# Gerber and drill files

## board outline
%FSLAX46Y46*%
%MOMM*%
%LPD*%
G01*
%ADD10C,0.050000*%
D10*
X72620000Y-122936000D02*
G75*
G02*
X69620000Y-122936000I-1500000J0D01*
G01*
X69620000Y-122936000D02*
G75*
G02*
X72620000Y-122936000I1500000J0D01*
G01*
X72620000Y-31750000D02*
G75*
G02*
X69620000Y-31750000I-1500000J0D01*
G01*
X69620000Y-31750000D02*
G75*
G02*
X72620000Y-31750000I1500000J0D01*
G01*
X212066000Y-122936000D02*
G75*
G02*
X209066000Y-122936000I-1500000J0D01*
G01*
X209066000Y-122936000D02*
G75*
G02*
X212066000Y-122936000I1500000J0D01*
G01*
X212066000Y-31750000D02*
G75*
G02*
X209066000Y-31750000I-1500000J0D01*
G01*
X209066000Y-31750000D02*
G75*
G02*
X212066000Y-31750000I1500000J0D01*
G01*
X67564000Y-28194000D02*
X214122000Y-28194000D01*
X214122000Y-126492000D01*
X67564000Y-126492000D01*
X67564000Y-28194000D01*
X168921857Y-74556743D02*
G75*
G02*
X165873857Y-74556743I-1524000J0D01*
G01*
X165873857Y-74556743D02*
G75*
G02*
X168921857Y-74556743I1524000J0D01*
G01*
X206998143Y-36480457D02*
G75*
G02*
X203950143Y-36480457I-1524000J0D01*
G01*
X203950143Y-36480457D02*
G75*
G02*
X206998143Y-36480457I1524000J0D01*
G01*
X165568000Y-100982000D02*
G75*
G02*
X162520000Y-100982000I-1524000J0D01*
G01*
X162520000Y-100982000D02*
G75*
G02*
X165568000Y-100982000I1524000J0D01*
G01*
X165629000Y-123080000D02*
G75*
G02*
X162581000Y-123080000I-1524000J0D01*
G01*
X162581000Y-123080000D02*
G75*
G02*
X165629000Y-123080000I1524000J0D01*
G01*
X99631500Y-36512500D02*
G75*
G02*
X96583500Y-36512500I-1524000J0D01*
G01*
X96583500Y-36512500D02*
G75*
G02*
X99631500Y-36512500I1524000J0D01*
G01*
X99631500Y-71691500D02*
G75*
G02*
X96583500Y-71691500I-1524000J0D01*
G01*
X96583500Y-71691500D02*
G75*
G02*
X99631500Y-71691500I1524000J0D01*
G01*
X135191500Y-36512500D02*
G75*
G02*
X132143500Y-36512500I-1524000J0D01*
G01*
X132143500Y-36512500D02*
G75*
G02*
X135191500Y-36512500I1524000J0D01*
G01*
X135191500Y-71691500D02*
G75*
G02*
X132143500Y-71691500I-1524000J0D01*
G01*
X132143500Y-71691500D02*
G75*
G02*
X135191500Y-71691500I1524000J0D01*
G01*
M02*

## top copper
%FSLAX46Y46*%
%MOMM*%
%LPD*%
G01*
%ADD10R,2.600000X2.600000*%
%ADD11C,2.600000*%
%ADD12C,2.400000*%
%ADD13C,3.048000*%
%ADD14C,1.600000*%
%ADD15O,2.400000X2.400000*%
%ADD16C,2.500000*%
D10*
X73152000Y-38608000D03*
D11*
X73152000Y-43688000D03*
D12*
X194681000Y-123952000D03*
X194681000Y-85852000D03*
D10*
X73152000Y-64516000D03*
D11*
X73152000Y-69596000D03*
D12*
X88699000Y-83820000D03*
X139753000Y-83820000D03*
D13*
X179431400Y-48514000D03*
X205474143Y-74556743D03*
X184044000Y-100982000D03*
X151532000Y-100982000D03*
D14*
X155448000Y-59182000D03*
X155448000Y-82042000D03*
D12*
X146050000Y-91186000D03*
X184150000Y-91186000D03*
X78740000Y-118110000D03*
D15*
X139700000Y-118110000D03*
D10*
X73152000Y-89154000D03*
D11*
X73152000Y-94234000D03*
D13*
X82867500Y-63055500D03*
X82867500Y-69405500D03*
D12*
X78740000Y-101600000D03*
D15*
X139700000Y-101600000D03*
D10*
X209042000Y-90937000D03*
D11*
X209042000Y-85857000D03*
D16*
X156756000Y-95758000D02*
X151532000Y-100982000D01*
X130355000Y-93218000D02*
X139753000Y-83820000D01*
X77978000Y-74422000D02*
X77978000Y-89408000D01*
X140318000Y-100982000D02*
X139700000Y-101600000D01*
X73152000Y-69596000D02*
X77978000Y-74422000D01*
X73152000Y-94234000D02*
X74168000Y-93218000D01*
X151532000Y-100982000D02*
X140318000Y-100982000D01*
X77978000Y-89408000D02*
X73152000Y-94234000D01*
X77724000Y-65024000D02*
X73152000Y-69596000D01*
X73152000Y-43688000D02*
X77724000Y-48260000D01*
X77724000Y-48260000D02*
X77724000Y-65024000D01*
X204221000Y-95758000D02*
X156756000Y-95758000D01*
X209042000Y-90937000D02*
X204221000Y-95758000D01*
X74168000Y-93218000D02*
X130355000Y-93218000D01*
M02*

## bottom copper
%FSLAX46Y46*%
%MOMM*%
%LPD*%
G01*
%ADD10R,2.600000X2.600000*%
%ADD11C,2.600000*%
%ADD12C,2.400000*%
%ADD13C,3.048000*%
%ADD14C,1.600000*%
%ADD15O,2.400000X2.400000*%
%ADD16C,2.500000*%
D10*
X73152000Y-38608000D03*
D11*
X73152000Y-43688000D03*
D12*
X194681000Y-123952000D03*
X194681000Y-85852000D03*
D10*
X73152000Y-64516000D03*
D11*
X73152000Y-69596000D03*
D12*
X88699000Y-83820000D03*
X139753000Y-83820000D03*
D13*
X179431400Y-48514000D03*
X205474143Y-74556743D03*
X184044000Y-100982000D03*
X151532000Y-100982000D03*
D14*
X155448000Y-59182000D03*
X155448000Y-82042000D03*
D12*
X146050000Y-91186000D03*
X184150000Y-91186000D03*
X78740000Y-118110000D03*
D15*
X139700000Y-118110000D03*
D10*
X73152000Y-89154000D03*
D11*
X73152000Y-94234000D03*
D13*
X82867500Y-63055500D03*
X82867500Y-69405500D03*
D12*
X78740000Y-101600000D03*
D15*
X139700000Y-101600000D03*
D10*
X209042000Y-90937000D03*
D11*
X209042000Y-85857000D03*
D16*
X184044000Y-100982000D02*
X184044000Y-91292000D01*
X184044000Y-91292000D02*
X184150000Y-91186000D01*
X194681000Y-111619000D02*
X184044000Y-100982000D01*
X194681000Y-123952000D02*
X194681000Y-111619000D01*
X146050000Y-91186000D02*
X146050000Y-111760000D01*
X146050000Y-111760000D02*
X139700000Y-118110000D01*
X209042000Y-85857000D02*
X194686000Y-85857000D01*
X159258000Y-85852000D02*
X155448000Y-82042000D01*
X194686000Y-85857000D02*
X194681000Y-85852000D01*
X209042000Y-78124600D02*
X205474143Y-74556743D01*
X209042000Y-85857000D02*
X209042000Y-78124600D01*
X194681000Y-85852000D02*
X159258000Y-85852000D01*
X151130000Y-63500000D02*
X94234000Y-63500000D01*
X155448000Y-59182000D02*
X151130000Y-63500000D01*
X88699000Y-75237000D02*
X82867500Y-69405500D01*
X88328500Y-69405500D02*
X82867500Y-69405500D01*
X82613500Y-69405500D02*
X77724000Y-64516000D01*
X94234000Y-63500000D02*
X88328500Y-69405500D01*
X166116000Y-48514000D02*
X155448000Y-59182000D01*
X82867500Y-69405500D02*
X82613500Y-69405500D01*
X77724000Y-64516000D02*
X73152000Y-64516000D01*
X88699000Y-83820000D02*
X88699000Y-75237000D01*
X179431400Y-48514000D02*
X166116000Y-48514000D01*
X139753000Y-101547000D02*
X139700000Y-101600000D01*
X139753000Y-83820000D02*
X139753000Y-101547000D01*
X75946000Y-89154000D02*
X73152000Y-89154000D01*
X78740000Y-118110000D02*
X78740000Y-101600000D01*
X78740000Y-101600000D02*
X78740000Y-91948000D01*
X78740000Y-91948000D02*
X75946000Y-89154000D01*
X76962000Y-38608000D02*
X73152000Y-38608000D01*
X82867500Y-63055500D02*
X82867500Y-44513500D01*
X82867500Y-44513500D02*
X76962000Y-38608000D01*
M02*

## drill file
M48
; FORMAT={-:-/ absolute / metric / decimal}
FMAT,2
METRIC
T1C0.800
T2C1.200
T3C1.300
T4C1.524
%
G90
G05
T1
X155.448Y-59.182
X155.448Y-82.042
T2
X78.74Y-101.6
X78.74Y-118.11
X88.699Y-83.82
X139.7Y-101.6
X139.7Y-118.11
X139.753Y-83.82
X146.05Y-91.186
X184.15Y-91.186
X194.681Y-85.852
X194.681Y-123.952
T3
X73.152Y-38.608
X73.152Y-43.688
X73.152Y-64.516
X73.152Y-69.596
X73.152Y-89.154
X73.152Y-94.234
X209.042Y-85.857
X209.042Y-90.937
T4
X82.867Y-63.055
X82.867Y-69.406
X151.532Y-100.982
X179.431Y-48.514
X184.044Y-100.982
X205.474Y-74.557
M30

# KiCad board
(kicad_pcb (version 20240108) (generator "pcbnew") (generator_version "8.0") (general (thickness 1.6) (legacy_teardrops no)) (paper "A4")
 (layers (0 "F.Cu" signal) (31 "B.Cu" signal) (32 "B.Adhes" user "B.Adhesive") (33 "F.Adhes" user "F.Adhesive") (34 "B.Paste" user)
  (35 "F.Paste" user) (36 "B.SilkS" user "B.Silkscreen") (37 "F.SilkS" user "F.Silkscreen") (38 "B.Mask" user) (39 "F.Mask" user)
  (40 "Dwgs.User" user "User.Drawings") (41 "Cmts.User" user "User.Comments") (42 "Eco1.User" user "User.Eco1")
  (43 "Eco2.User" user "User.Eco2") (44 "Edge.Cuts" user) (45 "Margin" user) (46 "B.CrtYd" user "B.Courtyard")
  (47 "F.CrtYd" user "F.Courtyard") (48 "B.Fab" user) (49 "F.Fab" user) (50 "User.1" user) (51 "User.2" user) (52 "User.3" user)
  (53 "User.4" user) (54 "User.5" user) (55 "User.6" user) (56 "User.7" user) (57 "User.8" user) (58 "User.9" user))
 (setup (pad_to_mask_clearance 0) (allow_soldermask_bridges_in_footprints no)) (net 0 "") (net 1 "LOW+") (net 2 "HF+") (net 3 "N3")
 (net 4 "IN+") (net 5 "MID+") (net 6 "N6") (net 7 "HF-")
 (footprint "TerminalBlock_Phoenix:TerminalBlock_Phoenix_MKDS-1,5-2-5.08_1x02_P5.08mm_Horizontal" (layer "F.Cu") (at 73.152 38.608 -90)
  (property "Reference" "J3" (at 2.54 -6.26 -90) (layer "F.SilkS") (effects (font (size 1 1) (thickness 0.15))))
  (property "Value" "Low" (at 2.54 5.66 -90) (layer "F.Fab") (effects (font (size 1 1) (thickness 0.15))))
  (pad "1" thru_hole rect (at 0 0 270) (size 2.6 2.6) (drill 1.3) (layers "*.Cu" "*.Mask") (remove_unused_layers no) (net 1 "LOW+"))
  (pad "2" thru_hole circle (at 5.08 0 270) (size 2.6 2.6) (drill 1.3) (layers "*.Cu" "*.Mask") (remove_unused_layers no) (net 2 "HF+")))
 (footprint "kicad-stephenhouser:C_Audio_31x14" (layer "F.Cu") (at 194.681 123.952 90)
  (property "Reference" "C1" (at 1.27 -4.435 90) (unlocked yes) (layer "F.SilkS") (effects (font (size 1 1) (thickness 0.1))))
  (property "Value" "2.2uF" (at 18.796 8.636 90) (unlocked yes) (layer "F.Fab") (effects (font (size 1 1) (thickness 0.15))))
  (pad "1" thru_hole circle (at 0 0 90) (size 2.4 2.4) (drill 1.2) (layers "*.Cu" "*.Mask") (remove_unused_layers no) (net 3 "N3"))
  (pad "2" thru_hole circle (at 38.1 0 90) (size 2.4 2.4) (drill 1.2) (layers "*.Cu" "*.Mask") (remove_unused_layers no) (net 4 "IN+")))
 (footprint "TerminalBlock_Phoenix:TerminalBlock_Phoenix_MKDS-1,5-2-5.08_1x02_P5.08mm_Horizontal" (layer "F.Cu") (at 73.152 64.516 -90)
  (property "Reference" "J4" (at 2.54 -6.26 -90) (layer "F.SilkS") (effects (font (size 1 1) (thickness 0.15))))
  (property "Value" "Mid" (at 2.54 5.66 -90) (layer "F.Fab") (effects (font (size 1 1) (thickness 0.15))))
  (pad "1" thru_hole rect (at 0 0 270) (size 2.6 2.6) (drill 1.3) (layers "*.Cu" "*.Mask") (remove_unused_layers no) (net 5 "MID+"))
  (pad "2" thru_hole circle (at 5.08 0 270) (size 2.6 2.6) (drill 1.3) (layers "*.Cu" "*.Mask") (remove_unused_layers no) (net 2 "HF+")))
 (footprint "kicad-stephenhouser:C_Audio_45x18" (layer "F.Cu") (at 88.699 83.82)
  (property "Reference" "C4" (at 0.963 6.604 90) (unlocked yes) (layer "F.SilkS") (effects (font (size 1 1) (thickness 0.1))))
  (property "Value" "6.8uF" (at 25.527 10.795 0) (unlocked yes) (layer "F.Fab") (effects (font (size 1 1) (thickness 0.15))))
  (pad "1" thru_hole circle (at 0 0) (size 2.4 2.4) (drill 1.2) (layers "*.Cu" "*.Mask") (remove_unused_layers no) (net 5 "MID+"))
  (pad "2" thru_hole circle (at 51.054 0) (size 2.4 2.4) (drill 1.2) (layers "*.Cu" "*.Mask") (remove_unused_layers no) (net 2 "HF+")))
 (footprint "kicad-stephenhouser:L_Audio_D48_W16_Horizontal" (layer "F.Cu") (at 186.436 55.5186 -45)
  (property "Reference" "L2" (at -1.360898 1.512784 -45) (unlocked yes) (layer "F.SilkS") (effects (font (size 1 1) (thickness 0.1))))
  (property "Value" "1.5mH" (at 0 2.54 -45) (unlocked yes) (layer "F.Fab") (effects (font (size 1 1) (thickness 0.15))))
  (fp_circle (center 0 26.924) (end 1.524 26.924) (stroke (width 0.05) (type default)) (fill none) (layer "Edge.Cuts"))
  (fp_circle (center 0 -26.924) (end 1.524 -26.924) (stroke (width 0.05) (type default)) (fill none) (layer "Edge.Cuts"))
  (pad "1" thru_hole circle (at -9.906 0 315) (size 3.048 3.048) (drill 1.524) (layers "*.Cu" "*.Mask") (remove_unused_layers no)
   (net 5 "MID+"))
  (pad "2" thru_hole circle (at 26.924 0 315) (size 3.048 3.048) (drill 1.524) (layers "*.Cu" "*.Mask") (remove_unused_layers no)
   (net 4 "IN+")))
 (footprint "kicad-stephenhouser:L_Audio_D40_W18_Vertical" (layer "F.Cu") (at 184.044 100.982 180)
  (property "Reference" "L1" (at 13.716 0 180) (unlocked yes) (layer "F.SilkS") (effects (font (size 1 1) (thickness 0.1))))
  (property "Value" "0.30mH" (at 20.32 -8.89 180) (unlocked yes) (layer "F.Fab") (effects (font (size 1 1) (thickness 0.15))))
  (fp_circle (center 20 0) (end 21.524 0) (stroke (width 0.05) (type default)) (fill none) (layer "Edge.Cuts"))
  (fp_circle (center 19.939 -22.098) (end 21.463 -22.098) (stroke (width 0.05) (type default)) (fill none) (layer "Edge.Cuts"))
  (pad "1" thru_hole circle (at 0 0 180) (size 3.048 3.048) (drill 1.524) (layers "*.Cu" "*.Mask") (remove_unused_layers no) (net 3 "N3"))
  (pad "2" thru_hole circle (at 32.512 0 180) (size 3.048 3.048) (drill 1.524) (layers "*.Cu" "*.Mask") (remove_unused_layers no)
   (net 2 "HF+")))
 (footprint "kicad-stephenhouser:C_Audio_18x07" (layer "F.Cu") (at 155.448 59.182 -90)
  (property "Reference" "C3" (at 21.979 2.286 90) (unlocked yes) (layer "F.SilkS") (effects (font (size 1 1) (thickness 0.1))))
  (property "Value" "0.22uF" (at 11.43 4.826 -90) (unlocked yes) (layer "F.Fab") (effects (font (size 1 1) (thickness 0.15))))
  (pad "1" thru_hole circle (at 0 0 270) (size 1.6 1.6) (drill 0.8) (layers "*.Cu" "*.Mask") (remove_unused_layers no) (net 5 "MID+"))
  (pad "2" thru_hole circle (at 22.86 0 270) (size 1.6 1.6) (drill 0.8) (layers "*.Cu" "*.Mask") (remove_unused_layers no) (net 4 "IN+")))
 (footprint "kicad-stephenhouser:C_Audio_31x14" (layer "F.Cu") (at 146.05 91.186)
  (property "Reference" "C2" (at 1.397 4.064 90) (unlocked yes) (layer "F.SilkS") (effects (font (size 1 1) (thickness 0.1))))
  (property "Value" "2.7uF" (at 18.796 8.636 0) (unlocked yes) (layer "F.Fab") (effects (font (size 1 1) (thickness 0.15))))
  (pad "1" thru_hole circle (at 0 0) (size 2.4 2.4) (drill 1.2) (layers "*.Cu" "*.Mask") (remove_unused_layers no) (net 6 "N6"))
  (pad "2" thru_hole circle (at 38.1 0) (size 2.4 2.4) (drill 1.2) (layers "*.Cu" "*.Mask") (remove_unused_layers no) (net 3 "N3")))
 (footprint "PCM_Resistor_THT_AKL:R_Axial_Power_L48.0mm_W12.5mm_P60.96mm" (layer "F.Cu") (at 78.74 118.11)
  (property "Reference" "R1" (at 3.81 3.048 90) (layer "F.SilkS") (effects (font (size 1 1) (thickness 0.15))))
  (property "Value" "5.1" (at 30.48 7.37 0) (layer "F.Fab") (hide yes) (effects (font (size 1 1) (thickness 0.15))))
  (pad "1" thru_hole circle (at 0 0) (size 2.4 2.4) (drill 1.2) (layers "*.Cu" "*.Mask") (remove_unused_layers no) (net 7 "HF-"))
  (pad "2" thru_hole oval (at 60.96 0) (size 2.4 2.4) (drill 1.2) (layers "*.Cu" "*.Mask") (remove_unused_layers no) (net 6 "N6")))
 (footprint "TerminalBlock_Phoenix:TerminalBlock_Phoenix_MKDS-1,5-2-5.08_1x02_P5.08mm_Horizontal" (layer "F.Cu") (at 73.152 89.154 -90)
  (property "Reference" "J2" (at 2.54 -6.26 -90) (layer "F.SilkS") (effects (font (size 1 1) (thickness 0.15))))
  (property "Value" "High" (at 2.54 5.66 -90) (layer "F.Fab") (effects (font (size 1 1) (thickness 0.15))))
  (pad "1" thru_hole rect (at 0 0 270) (size 2.6 2.6) (drill 1.3) (layers "*.Cu" "*.Mask") (remove_unused_layers no) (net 7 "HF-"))
  (pad "2" thru_hole circle (at 5.08 0 270) (size 2.6 2.6) (drill 1.3) (layers "*.Cu" "*.Mask") (remove_unused_layers no) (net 2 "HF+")))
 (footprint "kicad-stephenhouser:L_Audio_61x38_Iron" (layer "F.Cu") (at 82.8675 69.4055)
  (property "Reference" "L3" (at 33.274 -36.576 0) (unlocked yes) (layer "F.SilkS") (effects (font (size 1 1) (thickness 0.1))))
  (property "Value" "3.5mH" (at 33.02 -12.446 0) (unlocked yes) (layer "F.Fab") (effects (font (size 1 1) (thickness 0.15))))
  (fp_circle (center 15.24 -32.893) (end 16.764 -32.893) (stroke (width 0.05) (type default)) (fill none) (layer "Edge.Cuts"))
  (fp_circle (center 15.24 2.286) (end 16.764 2.286) (stroke (width 0.05) (type default)) (fill none) (layer "Edge.Cuts"))
  (fp_circle (center 50.8 -32.893) (end 52.324 -32.893) (stroke (width 0.05) (type default)) (fill none) (layer "Edge.Cuts"))
  (fp_circle (center 50.8 2.286) (end 52.324 2.286) (stroke (width 0.05) (type default)) (fill none) (layer "Edge.Cuts"))
  (pad "1" thru_hole circle (at 0 -6.35) (size 3.048 3.048) (drill 1.524) (layers "*.Cu" "*.Mask") (remove_unused_layers no) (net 1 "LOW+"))
  (pad "2" thru_hole circle (at 0 0) (size 3.048 3.048) (drill 1.524) (layers "*.Cu" "*.Mask") (remove_unused_layers no) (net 5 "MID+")))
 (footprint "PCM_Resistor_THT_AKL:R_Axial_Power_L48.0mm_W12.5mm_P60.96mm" (layer "F.Cu") (at 78.74 101.6)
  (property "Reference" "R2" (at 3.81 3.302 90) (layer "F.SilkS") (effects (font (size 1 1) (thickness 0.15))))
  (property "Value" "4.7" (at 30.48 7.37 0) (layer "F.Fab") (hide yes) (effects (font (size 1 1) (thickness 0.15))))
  (pad "1" thru_hole circle (at 0 0) (size 2.4 2.4) (drill 1.2) (layers "*.Cu" "*.Mask") (remove_unused_layers no) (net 7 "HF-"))
  (pad "2" thru_hole oval (at 60.96 0) (size 2.4 2.4) (drill 1.2) (layers "*.Cu" "*.Mask") (remove_unused_layers no) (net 2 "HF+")))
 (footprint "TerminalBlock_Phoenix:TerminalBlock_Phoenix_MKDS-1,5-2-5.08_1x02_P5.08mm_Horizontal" (layer "F.Cu") (at 209.042 90.937 90)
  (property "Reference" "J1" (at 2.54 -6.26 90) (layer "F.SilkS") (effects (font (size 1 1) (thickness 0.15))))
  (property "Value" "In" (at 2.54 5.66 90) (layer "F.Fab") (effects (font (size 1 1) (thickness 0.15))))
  (pad "1" thru_hole rect (at 0 0 90) (size 2.6 2.6) (drill 1.3) (layers "*.Cu" "*.Mask") (remove_unused_layers no) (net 2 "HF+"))
  (pad "2" thru_hole circle (at 5.08 0 90) (size 2.6 2.6) (drill 1.3) (layers "*.Cu" "*.Mask") (remove_unused_layers no) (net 4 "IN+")))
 (gr_circle (center 71.12 122.936) (end 72.62 122.936) (stroke (width 0.05) (type default)) (fill none) (layer "Edge.Cuts"))
 (gr_circle (center 71.12 31.75) (end 72.62 31.75) (stroke (width 0.05) (type default)) (fill none) (layer "Edge.Cuts"))
 (gr_circle (center 210.566 122.936) (end 212.066 122.936) (stroke (width 0.05) (type default)) (fill none) (layer "Edge.Cuts"))
 (gr_circle (center 210.566 31.75) (end 212.066 31.75) (stroke (width 0.05) (type default)) (fill none) (layer "Edge.Cuts"))
 (gr_rect (start 67.564 28.194) (end 214.122 126.492) (stroke (width 0.05) (type default)) (fill none) (layer "Edge.Cuts"))
 (segment (start 184.044 100.982) (end 184.044 91.292) (width 2.5) (layer "B.Cu") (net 3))
 (segment (start 184.044 91.292) (end 184.15 91.186) (width 2.5) (layer "B.Cu") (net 3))
 (segment (start 194.681 111.619) (end 184.044 100.982) (width 2.5) (layer "B.Cu") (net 3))
 (segment (start 194.681 123.952) (end 194.681 111.619) (width 2.5) (layer "B.Cu") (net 3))
 (segment (start 146.05 91.186) (end 146.05 111.76) (width 2.5) (layer "B.Cu") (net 6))
 (segment (start 146.05 111.76) (end 139.7 118.11) (width 2.5) (layer "B.Cu") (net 6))
 (segment (start 209.042 85.857) (end 194.686 85.857) (width 2.5) (layer "B.Cu") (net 4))
 (segment (start 159.258 85.852) (end 155.448 82.042) (width 2.5) (layer "B.Cu") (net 4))
 (segment (start 194.686 85.857) (end 194.681 85.852) (width 2.5) (layer "B.Cu") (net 4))
 (segment (start 209.042 78.1246) (end 205.474143 74.556743) (width 2.5) (layer "B.Cu") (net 4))
 (segment (start 209.042 85.857) (end 209.042 78.1246) (width 2.5) (layer "B.Cu") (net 4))
 (segment (start 194.681 85.852) (end 159.258 85.852) (width 2.5) (layer "B.Cu") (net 4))
 (segment (start 151.13 63.5) (end 94.234 63.5) (width 2.5) (layer "B.Cu") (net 5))
 (segment (start 155.448 59.182) (end 151.13 63.5) (width 2.5) (layer "B.Cu") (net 5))
 (segment (start 88.699 75.237) (end 82.8675 69.4055) (width 2.5) (layer "B.Cu") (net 5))
 (segment (start 88.3285 69.4055) (end 82.8675 69.4055) (width 2.5) (layer "B.Cu") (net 5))
 (segment (start 82.6135 69.4055) (end 77.724 64.516) (width 2.5) (layer "B.Cu") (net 5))
 (segment (start 94.234 63.5) (end 88.3285 69.4055) (width 2.5) (layer "B.Cu") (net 5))
 (segment (start 166.116 48.514) (end 155.448 59.182) (width 2.5) (layer "B.Cu") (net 5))
 (segment (start 82.8675 69.4055) (end 82.6135 69.4055) (width 2.5) (layer "B.Cu") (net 5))
 (segment (start 77.724 64.516) (end 73.152 64.516) (width 2.5) (layer "B.Cu") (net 5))
 (segment (start 88.699 83.82) (end 88.699 75.237) (width 2.5) (layer "B.Cu") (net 5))
 (segment (start 179.4314 48.514) (end 166.116 48.514) (width 2.5) (layer "B.Cu") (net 5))
 (segment (start 156.756 95.758) (end 151.532 100.982) (width 2.5) (layer "F.Cu") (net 2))
 (segment (start 130.355 93.218) (end 139.753 83.82) (width 2.5) (layer "F.Cu") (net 2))
 (segment (start 77.978 74.422) (end 77.978 89.408) (width 2.5) (layer "F.Cu") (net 2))
 (segment (start 140.318 100.982) (end 139.7 101.6) (width 2.5) (layer "F.Cu") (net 2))
 (segment (start 73.152 69.596) (end 77.978 74.422) (width 2.5) (layer "F.Cu") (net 2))
 (segment (start 73.152 94.234) (end 74.168 93.218) (width 2.5) (layer "F.Cu") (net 2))
 (segment (start 151.532 100.982) (end 140.318 100.982) (width 2.5) (layer "F.Cu") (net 2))
 (segment (start 77.978 89.408) (end 73.152 94.234) (width 2.5) (layer "F.Cu") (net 2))
 (segment (start 77.724 65.024) (end 73.152 69.596) (width 2.5) (layer "F.Cu") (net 2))
 (segment (start 73.152 43.688) (end 77.724 48.26) (width 2.5) (layer "F.Cu") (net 2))
 (segment (start 77.724 48.26) (end 77.724 65.024) (width 2.5) (layer "F.Cu") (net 2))
 (segment (start 204.221 95.758) (end 156.756 95.758) (width 2.5) (layer "F.Cu") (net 2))
 (segment (start 209.042 90.937) (end 204.221 95.758) (width 2.5) (layer "F.Cu") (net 2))
 (segment (start 74.168 93.218) (end 130.355 93.218) (width 2.5) (layer "F.Cu") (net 2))
 (segment (start 139.753 101.547) (end 139.7 101.6) (width 2.5) (layer "B.Cu") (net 2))
 (segment (start 139.753 83.82) (end 139.753 101.547) (width 2.5) (layer "B.Cu") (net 2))
 (segment (start 75.946 89.154) (end 73.152 89.154) (width 2.5) (layer "B.Cu") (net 7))
 (segment (start 78.74 118.11) (end 78.74 101.6) (width 2.5) (layer "B.Cu") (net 7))
 (segment (start 78.74 101.6) (end 78.74 91.948) (width 2.5) (layer "B.Cu") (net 7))
 (segment (start 78.74 91.948) (end 75.946 89.154) (width 2.5) (layer "B.Cu") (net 7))
 (segment (start 76.962 38.608) (end 73.152 38.608) (width 2.5) (layer "B.Cu") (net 1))
 (segment (start 82.8675 63.0555) (end 82.8675 44.5135) (width 2.5) (layer "B.Cu") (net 1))
 (segment (start 82.8675 44.5135) (end 76.962 38.608) (width 2.5) (layer "B.Cu") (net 1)))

